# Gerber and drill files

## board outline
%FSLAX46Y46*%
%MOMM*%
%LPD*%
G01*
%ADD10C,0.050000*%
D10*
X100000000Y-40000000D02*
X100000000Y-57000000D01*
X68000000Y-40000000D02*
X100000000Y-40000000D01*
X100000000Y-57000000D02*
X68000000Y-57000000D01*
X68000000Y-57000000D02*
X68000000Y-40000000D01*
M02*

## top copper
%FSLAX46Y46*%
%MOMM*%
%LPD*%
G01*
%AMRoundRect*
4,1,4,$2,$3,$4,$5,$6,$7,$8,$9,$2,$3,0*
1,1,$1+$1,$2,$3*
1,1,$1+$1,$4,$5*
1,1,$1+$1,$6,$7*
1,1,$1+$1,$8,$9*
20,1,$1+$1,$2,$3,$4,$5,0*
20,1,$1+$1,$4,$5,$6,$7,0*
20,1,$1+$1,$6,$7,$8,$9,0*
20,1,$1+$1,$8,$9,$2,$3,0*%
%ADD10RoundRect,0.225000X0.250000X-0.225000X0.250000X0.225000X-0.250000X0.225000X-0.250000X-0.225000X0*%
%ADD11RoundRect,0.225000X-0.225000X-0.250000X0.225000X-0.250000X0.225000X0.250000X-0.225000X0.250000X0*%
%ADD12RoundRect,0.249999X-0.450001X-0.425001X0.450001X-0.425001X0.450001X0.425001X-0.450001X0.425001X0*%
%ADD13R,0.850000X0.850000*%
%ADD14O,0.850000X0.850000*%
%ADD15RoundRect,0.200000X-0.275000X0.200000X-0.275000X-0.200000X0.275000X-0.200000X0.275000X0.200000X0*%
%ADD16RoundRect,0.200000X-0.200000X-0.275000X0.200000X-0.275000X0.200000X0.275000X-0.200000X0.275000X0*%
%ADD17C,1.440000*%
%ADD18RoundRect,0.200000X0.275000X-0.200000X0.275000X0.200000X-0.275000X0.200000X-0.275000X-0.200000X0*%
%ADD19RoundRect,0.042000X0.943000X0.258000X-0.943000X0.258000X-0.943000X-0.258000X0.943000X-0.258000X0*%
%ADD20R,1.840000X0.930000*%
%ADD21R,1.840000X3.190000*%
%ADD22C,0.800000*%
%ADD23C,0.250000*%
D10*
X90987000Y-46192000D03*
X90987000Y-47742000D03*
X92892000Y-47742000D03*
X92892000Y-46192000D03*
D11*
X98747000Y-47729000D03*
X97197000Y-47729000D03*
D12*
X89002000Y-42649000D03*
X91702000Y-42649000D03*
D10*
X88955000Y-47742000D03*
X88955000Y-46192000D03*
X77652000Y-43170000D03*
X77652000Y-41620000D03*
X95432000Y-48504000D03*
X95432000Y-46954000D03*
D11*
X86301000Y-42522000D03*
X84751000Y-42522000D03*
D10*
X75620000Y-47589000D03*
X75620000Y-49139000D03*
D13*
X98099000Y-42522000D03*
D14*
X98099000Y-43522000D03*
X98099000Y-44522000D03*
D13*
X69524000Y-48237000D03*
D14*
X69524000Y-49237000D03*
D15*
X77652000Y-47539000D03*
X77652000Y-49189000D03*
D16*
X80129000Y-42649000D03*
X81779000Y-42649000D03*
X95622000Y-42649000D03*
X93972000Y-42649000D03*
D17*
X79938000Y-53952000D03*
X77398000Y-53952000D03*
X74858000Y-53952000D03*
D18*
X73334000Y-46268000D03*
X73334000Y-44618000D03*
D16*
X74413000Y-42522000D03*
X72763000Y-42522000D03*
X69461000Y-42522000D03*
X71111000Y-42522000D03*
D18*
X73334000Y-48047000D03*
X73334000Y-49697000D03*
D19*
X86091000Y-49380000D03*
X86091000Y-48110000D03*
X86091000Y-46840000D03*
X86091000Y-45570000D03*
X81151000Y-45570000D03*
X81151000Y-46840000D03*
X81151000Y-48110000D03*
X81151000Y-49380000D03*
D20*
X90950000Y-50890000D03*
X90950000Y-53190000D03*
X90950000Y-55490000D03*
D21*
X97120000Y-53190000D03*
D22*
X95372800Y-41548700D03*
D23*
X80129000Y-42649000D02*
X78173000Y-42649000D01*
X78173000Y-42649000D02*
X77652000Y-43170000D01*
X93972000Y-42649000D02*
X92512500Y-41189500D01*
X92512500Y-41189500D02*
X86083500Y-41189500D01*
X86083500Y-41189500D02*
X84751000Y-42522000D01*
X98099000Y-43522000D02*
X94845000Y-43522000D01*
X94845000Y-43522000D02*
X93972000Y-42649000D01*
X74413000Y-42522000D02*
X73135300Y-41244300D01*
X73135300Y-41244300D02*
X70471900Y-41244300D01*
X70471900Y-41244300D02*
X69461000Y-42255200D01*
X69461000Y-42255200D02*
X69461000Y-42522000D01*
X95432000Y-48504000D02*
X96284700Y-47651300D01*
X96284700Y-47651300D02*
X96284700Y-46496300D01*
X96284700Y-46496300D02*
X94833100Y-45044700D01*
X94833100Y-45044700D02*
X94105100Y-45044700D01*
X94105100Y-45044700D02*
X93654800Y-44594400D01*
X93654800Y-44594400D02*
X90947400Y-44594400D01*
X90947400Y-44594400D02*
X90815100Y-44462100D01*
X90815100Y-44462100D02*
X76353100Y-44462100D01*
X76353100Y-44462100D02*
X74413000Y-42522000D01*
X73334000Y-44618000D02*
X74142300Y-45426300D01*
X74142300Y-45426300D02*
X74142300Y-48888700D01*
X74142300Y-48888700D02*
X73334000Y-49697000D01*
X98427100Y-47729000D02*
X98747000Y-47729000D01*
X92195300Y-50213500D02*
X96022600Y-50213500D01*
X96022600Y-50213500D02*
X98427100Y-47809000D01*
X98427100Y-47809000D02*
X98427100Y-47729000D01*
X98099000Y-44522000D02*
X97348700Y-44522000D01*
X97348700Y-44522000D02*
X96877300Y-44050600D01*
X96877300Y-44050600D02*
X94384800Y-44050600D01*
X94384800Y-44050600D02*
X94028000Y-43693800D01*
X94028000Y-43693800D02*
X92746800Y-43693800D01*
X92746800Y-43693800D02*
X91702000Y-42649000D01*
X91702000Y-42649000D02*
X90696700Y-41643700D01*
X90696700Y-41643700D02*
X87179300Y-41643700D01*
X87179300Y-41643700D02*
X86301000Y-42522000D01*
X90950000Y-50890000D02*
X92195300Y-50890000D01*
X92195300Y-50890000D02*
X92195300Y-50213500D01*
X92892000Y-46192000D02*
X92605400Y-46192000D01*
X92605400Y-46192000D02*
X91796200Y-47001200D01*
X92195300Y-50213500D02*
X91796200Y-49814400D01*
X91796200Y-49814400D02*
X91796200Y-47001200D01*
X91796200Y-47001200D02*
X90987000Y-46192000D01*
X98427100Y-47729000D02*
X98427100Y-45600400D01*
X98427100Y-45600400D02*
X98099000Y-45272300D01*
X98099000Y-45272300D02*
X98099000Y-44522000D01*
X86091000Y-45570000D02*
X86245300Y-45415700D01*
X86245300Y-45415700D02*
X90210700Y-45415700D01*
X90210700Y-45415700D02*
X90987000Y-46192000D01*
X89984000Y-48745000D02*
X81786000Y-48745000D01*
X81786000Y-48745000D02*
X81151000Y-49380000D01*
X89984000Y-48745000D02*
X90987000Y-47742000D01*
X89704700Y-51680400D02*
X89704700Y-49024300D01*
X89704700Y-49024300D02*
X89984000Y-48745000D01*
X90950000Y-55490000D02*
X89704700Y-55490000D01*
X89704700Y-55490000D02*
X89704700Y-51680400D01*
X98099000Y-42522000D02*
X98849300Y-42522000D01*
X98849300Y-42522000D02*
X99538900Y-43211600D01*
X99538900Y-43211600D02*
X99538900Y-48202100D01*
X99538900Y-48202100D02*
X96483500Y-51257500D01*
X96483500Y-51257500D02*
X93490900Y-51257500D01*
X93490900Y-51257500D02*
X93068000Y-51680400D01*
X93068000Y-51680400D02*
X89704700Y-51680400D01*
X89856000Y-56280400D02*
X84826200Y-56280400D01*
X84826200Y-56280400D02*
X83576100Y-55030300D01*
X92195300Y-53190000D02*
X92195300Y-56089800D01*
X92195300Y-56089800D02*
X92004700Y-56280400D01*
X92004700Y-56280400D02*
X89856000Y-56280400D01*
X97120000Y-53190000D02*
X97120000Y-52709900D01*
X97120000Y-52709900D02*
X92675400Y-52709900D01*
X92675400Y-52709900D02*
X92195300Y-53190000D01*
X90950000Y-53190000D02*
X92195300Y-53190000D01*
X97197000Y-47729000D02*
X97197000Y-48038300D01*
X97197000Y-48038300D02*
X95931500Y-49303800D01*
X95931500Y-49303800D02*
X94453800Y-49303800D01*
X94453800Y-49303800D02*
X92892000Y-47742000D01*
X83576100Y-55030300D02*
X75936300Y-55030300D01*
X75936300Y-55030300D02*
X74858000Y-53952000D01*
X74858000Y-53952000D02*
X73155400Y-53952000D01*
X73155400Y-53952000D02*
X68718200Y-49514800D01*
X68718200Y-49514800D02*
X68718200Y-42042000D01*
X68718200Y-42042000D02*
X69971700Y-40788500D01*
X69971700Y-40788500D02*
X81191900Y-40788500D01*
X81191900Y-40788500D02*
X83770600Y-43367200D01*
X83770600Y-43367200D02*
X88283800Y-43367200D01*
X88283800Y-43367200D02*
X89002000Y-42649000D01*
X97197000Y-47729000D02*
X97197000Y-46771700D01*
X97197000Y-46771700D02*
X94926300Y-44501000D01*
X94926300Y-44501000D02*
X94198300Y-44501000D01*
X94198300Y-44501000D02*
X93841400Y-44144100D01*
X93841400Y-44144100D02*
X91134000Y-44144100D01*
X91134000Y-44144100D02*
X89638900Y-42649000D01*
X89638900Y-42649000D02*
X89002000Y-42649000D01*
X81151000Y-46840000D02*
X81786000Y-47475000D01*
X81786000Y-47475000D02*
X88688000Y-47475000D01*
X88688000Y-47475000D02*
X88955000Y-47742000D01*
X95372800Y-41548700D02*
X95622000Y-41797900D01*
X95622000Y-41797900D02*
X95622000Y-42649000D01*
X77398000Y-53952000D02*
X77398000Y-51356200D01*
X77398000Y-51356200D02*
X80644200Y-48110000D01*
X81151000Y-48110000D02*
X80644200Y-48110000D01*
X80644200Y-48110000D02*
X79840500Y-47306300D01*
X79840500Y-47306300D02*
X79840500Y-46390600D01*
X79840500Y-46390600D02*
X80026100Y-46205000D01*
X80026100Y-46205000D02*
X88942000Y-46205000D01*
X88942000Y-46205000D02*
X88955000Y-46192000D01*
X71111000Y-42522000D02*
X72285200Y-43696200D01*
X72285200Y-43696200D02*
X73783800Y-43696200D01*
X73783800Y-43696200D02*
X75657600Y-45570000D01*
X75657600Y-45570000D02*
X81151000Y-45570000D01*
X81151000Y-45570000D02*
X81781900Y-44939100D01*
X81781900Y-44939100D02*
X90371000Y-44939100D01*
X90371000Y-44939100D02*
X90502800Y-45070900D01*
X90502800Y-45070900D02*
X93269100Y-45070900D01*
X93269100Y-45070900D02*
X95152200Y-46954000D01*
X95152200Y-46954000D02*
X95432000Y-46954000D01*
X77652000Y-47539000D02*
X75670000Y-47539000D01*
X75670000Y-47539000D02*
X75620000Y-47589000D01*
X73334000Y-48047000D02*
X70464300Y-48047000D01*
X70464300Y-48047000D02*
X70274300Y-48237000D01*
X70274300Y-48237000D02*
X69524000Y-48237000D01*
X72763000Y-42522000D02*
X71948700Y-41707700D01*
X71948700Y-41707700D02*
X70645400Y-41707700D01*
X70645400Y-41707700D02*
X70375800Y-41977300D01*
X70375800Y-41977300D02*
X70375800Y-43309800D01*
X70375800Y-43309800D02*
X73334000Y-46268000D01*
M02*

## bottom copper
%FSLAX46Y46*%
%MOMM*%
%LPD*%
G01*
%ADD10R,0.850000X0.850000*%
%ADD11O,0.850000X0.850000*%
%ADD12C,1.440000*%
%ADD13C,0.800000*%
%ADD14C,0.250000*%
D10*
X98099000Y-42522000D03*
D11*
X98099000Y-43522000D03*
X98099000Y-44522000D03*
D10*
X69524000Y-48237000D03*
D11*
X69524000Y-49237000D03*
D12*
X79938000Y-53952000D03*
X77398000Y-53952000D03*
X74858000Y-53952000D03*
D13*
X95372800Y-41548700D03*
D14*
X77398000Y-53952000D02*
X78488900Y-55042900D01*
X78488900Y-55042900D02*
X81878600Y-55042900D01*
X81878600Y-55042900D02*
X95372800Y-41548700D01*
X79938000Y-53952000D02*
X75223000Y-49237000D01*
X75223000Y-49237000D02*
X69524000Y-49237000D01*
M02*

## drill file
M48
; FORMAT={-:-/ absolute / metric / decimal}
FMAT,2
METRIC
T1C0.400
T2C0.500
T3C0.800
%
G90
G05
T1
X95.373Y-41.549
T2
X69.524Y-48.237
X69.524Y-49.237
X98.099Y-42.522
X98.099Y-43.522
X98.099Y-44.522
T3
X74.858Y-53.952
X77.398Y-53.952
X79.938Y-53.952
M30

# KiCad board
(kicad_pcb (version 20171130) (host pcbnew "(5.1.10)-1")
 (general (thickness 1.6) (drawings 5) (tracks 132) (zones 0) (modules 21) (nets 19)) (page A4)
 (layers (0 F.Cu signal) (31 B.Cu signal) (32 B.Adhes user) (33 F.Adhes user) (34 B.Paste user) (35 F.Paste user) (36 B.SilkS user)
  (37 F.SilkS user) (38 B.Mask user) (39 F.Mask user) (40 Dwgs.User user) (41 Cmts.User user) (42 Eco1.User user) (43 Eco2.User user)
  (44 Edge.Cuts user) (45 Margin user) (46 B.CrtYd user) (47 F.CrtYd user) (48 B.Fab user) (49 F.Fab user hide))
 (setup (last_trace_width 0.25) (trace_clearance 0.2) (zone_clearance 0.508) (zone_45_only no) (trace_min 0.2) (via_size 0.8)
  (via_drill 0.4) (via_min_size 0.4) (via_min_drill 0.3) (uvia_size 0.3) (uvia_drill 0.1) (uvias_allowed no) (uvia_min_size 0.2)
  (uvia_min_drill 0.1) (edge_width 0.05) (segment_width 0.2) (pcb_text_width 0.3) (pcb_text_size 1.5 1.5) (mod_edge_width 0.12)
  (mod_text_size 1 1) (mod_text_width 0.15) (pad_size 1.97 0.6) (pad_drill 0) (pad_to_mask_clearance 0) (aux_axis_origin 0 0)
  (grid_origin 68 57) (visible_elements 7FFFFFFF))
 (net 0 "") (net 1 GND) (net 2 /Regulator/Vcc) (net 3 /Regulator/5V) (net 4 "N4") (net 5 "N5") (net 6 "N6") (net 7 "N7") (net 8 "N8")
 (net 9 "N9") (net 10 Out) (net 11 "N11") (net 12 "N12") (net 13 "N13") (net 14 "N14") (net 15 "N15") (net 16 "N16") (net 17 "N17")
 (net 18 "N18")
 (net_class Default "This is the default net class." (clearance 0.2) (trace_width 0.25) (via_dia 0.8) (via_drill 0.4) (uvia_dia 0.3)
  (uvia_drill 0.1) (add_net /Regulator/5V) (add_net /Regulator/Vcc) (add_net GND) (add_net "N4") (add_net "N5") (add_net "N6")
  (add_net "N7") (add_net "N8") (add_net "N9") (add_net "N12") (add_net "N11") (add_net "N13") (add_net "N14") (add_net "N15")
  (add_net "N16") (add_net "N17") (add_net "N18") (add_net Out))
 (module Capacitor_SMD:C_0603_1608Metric (layer F.Cu) (at 90.987 46.967 90)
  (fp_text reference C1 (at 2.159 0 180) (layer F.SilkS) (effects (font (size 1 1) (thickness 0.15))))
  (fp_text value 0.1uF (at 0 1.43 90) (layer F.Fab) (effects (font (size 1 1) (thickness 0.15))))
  (pad 2 smd roundrect (at 0.775 0 90) (size 0.9 0.95) (layers F.Cu F.Paste F.Mask) (roundrect_rratio 0.25) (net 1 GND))
  (pad 1 smd roundrect (at -0.775 0 90) (size 0.9 0.95) (layers F.Cu F.Paste F.Mask) (roundrect_rratio 0.25) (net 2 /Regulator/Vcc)))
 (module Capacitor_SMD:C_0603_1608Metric (layer F.Cu) (at 92.892 46.967 90)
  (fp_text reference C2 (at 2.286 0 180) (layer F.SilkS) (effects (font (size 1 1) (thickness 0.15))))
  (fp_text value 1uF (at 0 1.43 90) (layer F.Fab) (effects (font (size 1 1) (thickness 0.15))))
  (pad 1 smd roundrect (at -0.775 0 90) (size 0.9 0.95) (layers F.Cu F.Paste F.Mask) (roundrect_rratio 0.25) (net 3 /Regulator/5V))
  (pad 2 smd roundrect (at 0.775 0 90) (size 0.9 0.95) (layers F.Cu F.Paste F.Mask) (roundrect_rratio 0.25) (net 1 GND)))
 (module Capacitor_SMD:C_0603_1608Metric (layer F.Cu) (at 97.972 47.729)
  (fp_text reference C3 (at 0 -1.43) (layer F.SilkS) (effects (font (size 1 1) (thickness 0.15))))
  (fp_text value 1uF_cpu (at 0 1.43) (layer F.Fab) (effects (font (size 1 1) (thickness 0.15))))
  (pad 2 smd roundrect (at 0.775 0) (size 0.9 0.95) (layers F.Cu F.Paste F.Mask) (roundrect_rratio 0.25) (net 1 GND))
  (pad 1 smd roundrect (at -0.775 0) (size 0.9 0.95) (layers F.Cu F.Paste F.Mask) (roundrect_rratio 0.25) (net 3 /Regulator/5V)))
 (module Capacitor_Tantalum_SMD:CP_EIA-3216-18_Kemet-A (layer F.Cu) (at 90.352 42.649)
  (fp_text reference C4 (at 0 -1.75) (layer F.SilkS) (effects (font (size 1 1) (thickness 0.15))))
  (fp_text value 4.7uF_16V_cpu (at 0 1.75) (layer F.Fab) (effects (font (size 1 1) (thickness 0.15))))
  (pad 1 smd roundrect (at -1.35 0) (size 1.4 1.35) (layers F.Cu F.Paste F.Mask) (roundrect_rratio 0.1851844444444445) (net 3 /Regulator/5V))
  (pad 2 smd roundrect (at 1.35 0) (size 1.4 1.35) (layers F.Cu F.Paste F.Mask) (roundrect_rratio 0.1851844444444445) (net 1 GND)))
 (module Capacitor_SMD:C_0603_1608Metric (layer F.Cu) (at 88.955 46.967 90)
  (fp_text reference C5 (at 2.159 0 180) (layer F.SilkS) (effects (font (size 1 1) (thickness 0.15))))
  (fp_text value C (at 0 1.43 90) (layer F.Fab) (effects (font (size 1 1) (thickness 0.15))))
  (pad 1 smd roundrect (at -0.775 0 90) (size 0.9 0.95) (layers F.Cu F.Paste F.Mask) (roundrect_rratio 0.25) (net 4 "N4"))
  (pad 2 smd roundrect (at 0.775 0 90) (size 0.9 0.95) (layers F.Cu F.Paste F.Mask) (roundrect_rratio 0.25) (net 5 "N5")))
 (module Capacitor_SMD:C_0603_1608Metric (layer F.Cu) (at 77.652 42.395 90)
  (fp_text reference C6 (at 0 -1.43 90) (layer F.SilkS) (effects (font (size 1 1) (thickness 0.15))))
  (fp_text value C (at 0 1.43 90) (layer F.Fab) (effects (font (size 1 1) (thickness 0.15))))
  (pad 1 smd roundrect (at -0.775 0 90) (size 0.9 0.95) (layers F.Cu F.Paste F.Mask) (roundrect_rratio 0.25) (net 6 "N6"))
  (pad 2 smd roundrect (at 0.775 0 90) (size 0.9 0.95) (layers F.Cu F.Paste F.Mask) (roundrect_rratio 0.25) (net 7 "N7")))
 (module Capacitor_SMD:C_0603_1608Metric (layer F.Cu) (at 95.432 47.729 90)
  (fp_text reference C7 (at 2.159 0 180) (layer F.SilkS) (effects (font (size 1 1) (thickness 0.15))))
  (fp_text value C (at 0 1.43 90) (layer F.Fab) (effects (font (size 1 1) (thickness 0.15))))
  (pad 1 smd roundrect (at -0.775 0 90) (size 0.9 0.95) (layers F.Cu F.Paste F.Mask) (roundrect_rratio 0.25) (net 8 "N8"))
  (pad 2 smd roundrect (at 0.775 0 90) (size 0.9 0.95) (layers F.Cu F.Paste F.Mask) (roundrect_rratio 0.25) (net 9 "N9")))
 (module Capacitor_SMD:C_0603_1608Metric (layer F.Cu) (at 85.526 42.522)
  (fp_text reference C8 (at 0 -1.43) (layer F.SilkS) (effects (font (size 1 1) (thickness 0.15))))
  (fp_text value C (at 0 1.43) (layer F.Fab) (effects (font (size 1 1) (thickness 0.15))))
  (pad 2 smd roundrect (at 0.775 0) (size 0.9 0.95) (layers F.Cu F.Paste F.Mask) (roundrect_rratio 0.25) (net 1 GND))
  (pad 1 smd roundrect (at -0.775 0) (size 0.9 0.95) (layers F.Cu F.Paste F.Mask) (roundrect_rratio 0.25) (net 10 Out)))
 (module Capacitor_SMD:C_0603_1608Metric (layer F.Cu) (at 75.62 48.364 90)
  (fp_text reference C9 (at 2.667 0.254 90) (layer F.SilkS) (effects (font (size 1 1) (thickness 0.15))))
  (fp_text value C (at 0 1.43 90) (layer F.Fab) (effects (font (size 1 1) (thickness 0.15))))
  (pad 2 smd roundrect (at 0.775 0 90) (size 0.9 0.95) (layers F.Cu F.Paste F.Mask) (roundrect_rratio 0.25) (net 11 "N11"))
  (pad 1 smd roundrect (at -0.775 0 90) (size 0.9 0.95) (layers F.Cu F.Paste F.Mask) (roundrect_rratio 0.25) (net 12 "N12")))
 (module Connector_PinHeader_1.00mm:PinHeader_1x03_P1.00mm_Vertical (layer F.Cu) (at 98.099 42.522)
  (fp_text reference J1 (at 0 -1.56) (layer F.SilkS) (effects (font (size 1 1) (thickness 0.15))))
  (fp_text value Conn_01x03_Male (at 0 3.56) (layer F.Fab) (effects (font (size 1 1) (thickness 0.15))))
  (pad 1 thru_hole rect (at 0 0) (size 0.85 0.85) (drill 0.5) (layers *.Cu *.Mask) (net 2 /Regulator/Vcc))
  (pad 2 thru_hole oval (at 0 1) (size 0.85 0.85) (drill 0.5) (layers *.Cu *.Mask) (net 10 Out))
  (pad 3 thru_hole oval (at 0 2) (size 0.85 0.85) (drill 0.5) (layers *.Cu *.Mask) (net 1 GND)))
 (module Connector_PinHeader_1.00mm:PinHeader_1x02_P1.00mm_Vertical (layer F.Cu) (at 69.524 48.237)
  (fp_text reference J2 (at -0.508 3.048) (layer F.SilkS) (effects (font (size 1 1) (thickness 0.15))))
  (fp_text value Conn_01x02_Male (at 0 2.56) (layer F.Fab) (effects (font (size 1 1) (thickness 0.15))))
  (pad 1 thru_hole rect (at 0 0) (size 0.85 0.85) (drill 0.5) (layers *.Cu *.Mask) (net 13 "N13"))
  (pad 2 thru_hole oval (at 0 1) (size 0.85 0.85) (drill 0.5) (layers *.Cu *.Mask) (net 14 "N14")))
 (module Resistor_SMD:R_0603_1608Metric (layer F.Cu) (at 77.652 48.364 270)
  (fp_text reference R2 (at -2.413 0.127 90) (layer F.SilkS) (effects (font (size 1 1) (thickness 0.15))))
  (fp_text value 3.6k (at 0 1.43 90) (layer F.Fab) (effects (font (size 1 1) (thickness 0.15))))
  (pad 1 smd roundrect (at -0.825 0 270) (size 0.8 0.95) (layers F.Cu F.Paste F.Mask) (roundrect_rratio 0.25) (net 11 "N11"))
  (pad 2 smd roundrect (at 0.825 0 270) (size 0.8 0.95) (layers F.Cu F.Paste F.Mask) (roundrect_rratio 0.25) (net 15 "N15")))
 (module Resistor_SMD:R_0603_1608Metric (layer F.Cu) (at 80.954 42.649)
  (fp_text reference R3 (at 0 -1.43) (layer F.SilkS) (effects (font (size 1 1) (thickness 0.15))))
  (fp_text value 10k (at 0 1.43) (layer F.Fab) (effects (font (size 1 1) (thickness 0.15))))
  (pad 1 smd roundrect (at -0.825 0) (size 0.8 0.95) (layers F.Cu F.Paste F.Mask) (roundrect_rratio 0.25) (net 6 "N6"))
  (pad 2 smd roundrect (at 0.825 0) (size 0.8 0.95) (layers F.Cu F.Paste F.Mask) (roundrect_rratio 0.25) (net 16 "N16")))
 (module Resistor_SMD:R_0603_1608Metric (layer F.Cu) (at 94.797 42.649)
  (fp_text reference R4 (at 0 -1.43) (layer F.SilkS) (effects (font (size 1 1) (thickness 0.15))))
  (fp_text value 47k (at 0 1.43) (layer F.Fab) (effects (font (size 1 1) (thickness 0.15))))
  (pad 2 smd roundrect (at 0.825 0) (size 0.8 0.95) (layers F.Cu F.Paste F.Mask) (roundrect_rratio 0.25) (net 5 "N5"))
  (pad 1 smd roundrect (at -0.825 0) (size 0.8 0.95) (layers F.Cu F.Paste F.Mask) (roundrect_rratio 0.25) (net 10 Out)))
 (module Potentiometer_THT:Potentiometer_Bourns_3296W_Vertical (layer F.Cu) (at 79.938 53.952)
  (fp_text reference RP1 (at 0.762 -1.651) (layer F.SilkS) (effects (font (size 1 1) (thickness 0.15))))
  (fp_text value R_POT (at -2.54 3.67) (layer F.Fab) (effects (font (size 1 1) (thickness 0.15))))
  (pad 1 thru_hole circle (at 0 0) (size 1.44 1.44) (drill 0.8) (layers *.Cu *.Mask) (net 14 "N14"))
  (pad 2 thru_hole circle (at -2.54 0) (size 1.44 1.44) (drill 0.8) (layers *.Cu *.Mask) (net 5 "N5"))
  (pad 3 thru_hole circle (at -5.08 0) (size 1.44 1.44) (drill 0.8) (layers *.Cu *.Mask) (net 3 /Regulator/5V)))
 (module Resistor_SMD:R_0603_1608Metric (layer F.Cu) (at 73.334 45.443 90)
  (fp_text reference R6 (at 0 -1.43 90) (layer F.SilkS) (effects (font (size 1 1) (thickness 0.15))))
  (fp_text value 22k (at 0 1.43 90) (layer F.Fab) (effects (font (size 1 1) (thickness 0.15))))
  (pad 1 smd roundrect (at -0.825 0 90) (size 0.8 0.95) (layers F.Cu F.Paste F.Mask) (roundrect_rratio 0.25) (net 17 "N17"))
  (pad 2 smd roundrect (at 0.825 0 90) (size 0.8 0.95) (layers F.Cu F.Paste F.Mask) (roundrect_rratio 0.25) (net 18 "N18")))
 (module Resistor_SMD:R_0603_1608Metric (layer F.Cu) (at 73.588 42.522)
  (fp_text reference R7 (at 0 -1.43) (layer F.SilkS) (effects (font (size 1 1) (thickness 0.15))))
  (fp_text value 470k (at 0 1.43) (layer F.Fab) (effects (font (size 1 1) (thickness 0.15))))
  (pad 2 smd roundrect (at 0.825 0) (size 0.8 0.95) (layers F.Cu F.Paste F.Mask) (roundrect_rratio 0.25) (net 8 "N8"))
  (pad 1 smd roundrect (at -0.825 0) (size 0.8 0.95) (layers F.Cu F.Paste F.Mask) (roundrect_rratio 0.25) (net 17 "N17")))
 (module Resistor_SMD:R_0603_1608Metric (layer F.Cu) (at 70.286 42.522)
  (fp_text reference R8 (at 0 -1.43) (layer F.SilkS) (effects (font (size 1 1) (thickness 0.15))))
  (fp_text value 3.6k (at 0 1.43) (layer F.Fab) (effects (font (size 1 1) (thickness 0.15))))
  (pad 1 smd roundrect (at -0.825 0) (size 0.8 0.95) (layers F.Cu F.Paste F.Mask) (roundrect_rratio 0.25) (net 8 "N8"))
  (pad 2 smd roundrect (at 0.825 0) (size 0.8 0.95) (layers F.Cu F.Paste F.Mask) (roundrect_rratio 0.25) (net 9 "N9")))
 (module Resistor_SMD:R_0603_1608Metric (layer F.Cu) (at 73.334 48.872 90)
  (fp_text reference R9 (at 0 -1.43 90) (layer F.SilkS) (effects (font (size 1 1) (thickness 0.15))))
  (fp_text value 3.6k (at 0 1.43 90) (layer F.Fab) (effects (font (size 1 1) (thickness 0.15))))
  (pad 2 smd roundrect (at 0.825 0 90) (size 0.8 0.95) (layers F.Cu F.Paste F.Mask) (roundrect_rratio 0.25) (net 13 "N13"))
  (pad 1 smd roundrect (at -0.825 0 90) (size 0.8 0.95) (layers F.Cu F.Paste F.Mask) (roundrect_rratio 0.25) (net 18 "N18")))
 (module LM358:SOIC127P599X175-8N (layer F.Cu) (at 83.621 47.475 180)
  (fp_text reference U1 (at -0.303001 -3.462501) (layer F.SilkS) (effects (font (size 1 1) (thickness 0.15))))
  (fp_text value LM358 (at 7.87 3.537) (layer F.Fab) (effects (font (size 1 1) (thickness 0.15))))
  (pad 1 smd roundrect (at -2.47 -1.905 180) (size 1.97 0.6) (layers F.Cu F.Paste F.Mask) (roundrect_rratio 0.07000000000000001))
  (pad 2 smd roundrect (at -2.47 -0.635 180) (size 1.97 0.6) (layers F.Cu F.Paste F.Mask) (roundrect_rratio 0.07000000000000001))
  (pad 3 smd roundrect (at -2.47 0.635 180) (size 1.97 0.6) (layers F.Cu F.Paste F.Mask) (roundrect_rratio 0.07000000000000001))
  (pad 4 smd roundrect (at -2.47 1.905 180) (size 1.97 0.6) (layers F.Cu F.Paste F.Mask) (roundrect_rratio 0.07000000000000001) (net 1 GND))
  (pad 5 smd roundrect (at 2.47 1.905 180) (size 1.97 0.6) (layers F.Cu F.Paste F.Mask) (roundrect_rratio 0.07000000000000001) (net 9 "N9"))
  (pad 6 smd roundrect (at 2.47 0.635 180) (size 1.97 0.6) (layers F.Cu F.Paste F.Mask) (roundrect_rratio 0.07000000000000001) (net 4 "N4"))
  (pad 7 smd roundrect (at 2.47 -0.635 180) (size 1.97 0.6) (layers F.Cu F.Paste F.Mask) (roundrect_rratio 0.07000000000000001) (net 5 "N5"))
  (pad 8 smd roundrect (at 2.47 -1.905 180) (size 1.97 0.6) (layers F.Cu F.Paste F.Mask) (roundrect_rratio 0.07000000000000001)
   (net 2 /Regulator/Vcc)))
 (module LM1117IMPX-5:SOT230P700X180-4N (layer F.Cu) (at 94.035 53.19)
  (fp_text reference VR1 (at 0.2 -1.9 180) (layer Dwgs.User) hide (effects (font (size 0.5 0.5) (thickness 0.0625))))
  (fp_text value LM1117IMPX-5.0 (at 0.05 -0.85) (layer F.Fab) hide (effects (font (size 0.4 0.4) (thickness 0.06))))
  (pad 1 smd rect (at -3.085 -2.3) (size 1.84 0.93) (layers F.Cu F.Paste F.Mask) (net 1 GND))
  (pad 2 smd rect (at -3.085 0) (size 1.84 0.93) (layers F.Cu F.Paste F.Mask) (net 3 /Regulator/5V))
  (pad 3 smd rect (at -3.085 2.3) (size 1.84 0.93) (layers F.Cu F.Paste F.Mask) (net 2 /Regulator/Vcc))
  (pad 4 smd rect (at 3.085 0) (size 1.84 3.19) (layers F.Cu F.Paste F.Mask) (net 3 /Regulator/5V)))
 (gr_line (start 100 40) (end 100 57) (layer Edge.Cuts) (width 0.05))
 (gr_line (start 68 40) (end 100 40) (layer Edge.Cuts) (width 0.05))
 (gr_line (start 100 57) (end 68 57) (layer Edge.Cuts) (width 0.05))
 (gr_line (start 68 57) (end 68 40) (layer Edge.Cuts) (width 0.05))
 (segment (start 80.129 42.649) (end 78.173 42.649) (width 0.25) (layer F.Cu) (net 6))
 (segment (start 78.173 42.649) (end 77.652 43.17) (width 0.25) (layer F.Cu) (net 6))
 (segment (start 93.972 42.649) (end 92.5125 41.1895) (width 0.25) (layer F.Cu) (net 10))
 (segment (start 92.5125 41.1895) (end 86.0835 41.1895) (width 0.25) (layer F.Cu) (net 10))
 (segment (start 86.0835 41.1895) (end 84.751 42.522) (width 0.25) (layer F.Cu) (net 10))
 (segment (start 98.099 43.522) (end 94.845 43.522) (width 0.25) (layer F.Cu) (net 10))
 (segment (start 94.845 43.522) (end 93.972 42.649) (width 0.25) (layer F.Cu) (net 10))
 (segment (start 74.413 42.522) (end 73.1353 41.2443) (width 0.25) (layer F.Cu) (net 8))
 (segment (start 73.1353 41.2443) (end 70.4719 41.2443) (width 0.25) (layer F.Cu) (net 8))
 (segment (start 70.4719 41.2443) (end 69.461 42.2552) (width 0.25) (layer F.Cu) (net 8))
 (segment (start 69.461 42.2552) (end 69.461 42.522) (width 0.25) (layer F.Cu) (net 8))
 (segment (start 95.432 48.504) (end 96.2847 47.6513) (width 0.25) (layer F.Cu) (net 8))
 (segment (start 96.2847 47.6513) (end 96.2847 46.4963) (width 0.25) (layer F.Cu) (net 8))
 (segment (start 96.2847 46.4963) (end 94.8331 45.0447) (width 0.25) (layer F.Cu) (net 8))
 (segment (start 94.8331 45.0447) (end 94.1051 45.0447) (width 0.25) (layer F.Cu) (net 8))
 (segment (start 94.1051 45.0447) (end 93.6548 44.5944) (width 0.25) (layer F.Cu) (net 8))
 (segment (start 93.6548 44.5944) (end 90.9474 44.5944) (width 0.25) (layer F.Cu) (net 8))
 (segment (start 90.9474 44.5944) (end 90.8151 44.4621) (width 0.25) (layer F.Cu) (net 8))
 (segment (start 90.8151 44.4621) (end 76.3531 44.4621) (width 0.25) (layer F.Cu) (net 8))
 (segment (start 76.3531 44.4621) (end 74.413 42.522) (width 0.25) (layer F.Cu) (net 8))
 (segment (start 73.334 44.618) (end 74.1423 45.4263) (width 0.25) (layer F.Cu) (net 18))
 (segment (start 74.1423 45.4263) (end 74.1423 48.8887) (width 0.25) (layer F.Cu) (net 18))
 (segment (start 74.1423 48.8887) (end 73.334 49.697) (width 0.25) (layer F.Cu) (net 18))
 (segment (start 98.4271 47.729) (end 98.747 47.729) (width 0.25) (layer F.Cu) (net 1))
 (segment (start 92.1953 50.2135) (end 96.0226 50.2135) (width 0.25) (layer F.Cu) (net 1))
 (segment (start 96.0226 50.2135) (end 98.4271 47.809) (width 0.25) (layer F.Cu) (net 1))
 (segment (start 98.4271 47.809) (end 98.4271 47.729) (width 0.25) (layer F.Cu) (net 1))
 (segment (start 98.099 44.522) (end 97.3487 44.522) (width 0.25) (layer F.Cu) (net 1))
 (segment (start 97.3487 44.522) (end 96.8773 44.0506) (width 0.25) (layer F.Cu) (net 1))
 (segment (start 96.8773 44.0506) (end 94.3848 44.0506) (width 0.25) (layer F.Cu) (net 1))
 (segment (start 94.3848 44.0506) (end 94.028 43.6938) (width 0.25) (layer F.Cu) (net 1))
 (segment (start 94.028 43.6938) (end 92.7468 43.6938) (width 0.25) (layer F.Cu) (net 1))
 (segment (start 92.7468 43.6938) (end 91.702 42.649) (width 0.25) (layer F.Cu) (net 1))
 (segment (start 91.702 42.649) (end 90.6967 41.6437) (width 0.25) (layer F.Cu) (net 1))
 (segment (start 90.6967 41.6437) (end 87.1793 41.6437) (width 0.25) (layer F.Cu) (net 1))
 (segment (start 87.1793 41.6437) (end 86.301 42.522) (width 0.25) (layer F.Cu) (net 1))
 (segment (start 90.95 50.89) (end 92.1953 50.89) (width 0.25) (layer F.Cu) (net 1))
 (segment (start 92.1953 50.89) (end 92.1953 50.2135) (width 0.25) (layer F.Cu) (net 1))
 (segment (start 92.892 46.192) (end 92.6054 46.192) (width 0.25) (layer F.Cu) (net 1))
 (segment (start 92.6054 46.192) (end 91.7962 47.0012) (width 0.25) (layer F.Cu) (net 1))
 (segment (start 92.1953 50.2135) (end 91.7962 49.8144) (width 0.25) (layer F.Cu) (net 1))
 (segment (start 91.7962 49.8144) (end 91.7962 47.0012) (width 0.25) (layer F.Cu) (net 1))
 (segment (start 91.7962 47.0012) (end 90.987 46.192) (width 0.25) (layer F.Cu) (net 1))
 (segment (start 98.4271 47.729) (end 98.4271 45.6004) (width 0.25) (layer F.Cu) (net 1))
 (segment (start 98.4271 45.6004) (end 98.099 45.2723) (width 0.25) (layer F.Cu) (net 1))
 (segment (start 98.099 45.2723) (end 98.099 44.522) (width 0.25) (layer F.Cu) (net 1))
 (segment (start 86.091 45.57) (end 86.2453 45.4157) (width 0.25) (layer F.Cu) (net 1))
 (segment (start 86.2453 45.4157) (end 90.2107 45.4157) (width 0.25) (layer F.Cu) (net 1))
 (segment (start 90.2107 45.4157) (end 90.987 46.192) (width 0.25) (layer F.Cu) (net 1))
 (segment (start 89.984 48.745) (end 81.786 48.745) (width 0.25) (layer F.Cu) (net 2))
 (segment (start 81.786 48.745) (end 81.151 49.38) (width 0.25) (layer F.Cu) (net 2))
 (segment (start 89.984 48.745) (end 90.987 47.742) (width 0.25) (layer F.Cu) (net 2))
 (segment (start 89.7047 51.6804) (end 89.7047 49.0243) (width 0.25) (layer F.Cu) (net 2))
 (segment (start 89.7047 49.0243) (end 89.984 48.745) (width 0.25) (layer F.Cu) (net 2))
 (segment (start 90.95 55.49) (end 89.7047 55.49) (width 0.25) (layer F.Cu) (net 2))
 (segment (start 89.7047 55.49) (end 89.7047 51.6804) (width 0.25) (layer F.Cu) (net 2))
 (segment (start 98.099 42.522) (end 98.8493 42.522) (width 0.25) (layer F.Cu) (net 2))
 (segment (start 98.8493 42.522) (end 99.5389 43.2116) (width 0.25) (layer F.Cu) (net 2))
 (segment (start 99.5389 43.2116) (end 99.5389 48.2021) (width 0.25) (layer F.Cu) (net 2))
 (segment (start 99.5389 48.2021) (end 96.4835 51.2575) (width 0.25) (layer F.Cu) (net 2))
 (segment (start 96.4835 51.2575) (end 93.4909 51.2575) (width 0.25) (layer F.Cu) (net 2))
 (segment (start 93.4909 51.2575) (end 93.068 51.6804) (width 0.25) (layer F.Cu) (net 2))
 (segment (start 93.068 51.6804) (end 89.7047 51.6804) (width 0.25) (layer F.Cu) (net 2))
 (segment (start 89.856 56.2804) (end 84.8262 56.2804) (width 0.25) (layer F.Cu) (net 3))
 (segment (start 84.8262 56.2804) (end 83.5761 55.0303) (width 0.25) (layer F.Cu) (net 3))
 (segment (start 92.1953 53.19) (end 92.1953 56.0898) (width 0.25) (layer F.Cu) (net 3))
 (segment (start 92.1953 56.0898) (end 92.0047 56.2804) (width 0.25) (layer F.Cu) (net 3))
 (segment (start 92.0047 56.2804) (end 89.856 56.2804) (width 0.25) (layer F.Cu) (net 3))
 (segment (start 97.12 53.19) (end 97.12 52.7099) (width 0.25) (layer F.Cu) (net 3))
 (segment (start 97.12 52.7099) (end 92.6754 52.7099) (width 0.25) (layer F.Cu) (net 3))
 (segment (start 92.6754 52.7099) (end 92.1953 53.19) (width 0.25) (layer F.Cu) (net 3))
 (segment (start 90.95 53.19) (end 92.1953 53.19) (width 0.25) (layer F.Cu) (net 3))
 (segment (start 97.197 47.729) (end 97.197 48.0383) (width 0.25) (layer F.Cu) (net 3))
 (segment (start 97.197 48.0383) (end 95.9315 49.3038) (width 0.25) (layer F.Cu) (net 3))
 (segment (start 95.9315 49.3038) (end 94.4538 49.3038) (width 0.25) (layer F.Cu) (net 3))
 (segment (start 94.4538 49.3038) (end 92.892 47.742) (width 0.25) (layer F.Cu) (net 3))
 (segment (start 83.5761 55.0303) (end 75.9363 55.0303) (width 0.25) (layer F.Cu) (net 3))
 (segment (start 75.9363 55.0303) (end 74.858 53.952) (width 0.25) (layer F.Cu) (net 3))
 (segment (start 74.858 53.952) (end 73.1554 53.952) (width 0.25) (layer F.Cu) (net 3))
 (segment (start 73.1554 53.952) (end 68.7182 49.5148) (width 0.25) (layer F.Cu) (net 3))
 (segment (start 68.7182 49.5148) (end 68.7182 42.042) (width 0.25) (layer F.Cu) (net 3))
 (segment (start 68.7182 42.042) (end 69.9717 40.7885) (width 0.25) (layer F.Cu) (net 3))
 (segment (start 69.9717 40.7885) (end 81.1919 40.7885) (width 0.25) (layer F.Cu) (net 3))
 (segment (start 81.1919 40.7885) (end 83.7706 43.3672) (width 0.25) (layer F.Cu) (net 3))
 (segment (start 83.7706 43.3672) (end 88.2838 43.3672) (width 0.25) (layer F.Cu) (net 3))
 (segment (start 88.2838 43.3672) (end 89.002 42.649) (width 0.25) (layer F.Cu) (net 3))
 (segment (start 97.197 47.729) (end 97.197 46.7717) (width 0.25) (layer F.Cu) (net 3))
 (segment (start 97.197 46.7717) (end 94.9263 44.501) (width 0.25) (layer F.Cu) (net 3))
 (segment (start 94.9263 44.501) (end 94.1983 44.501) (width 0.25) (layer F.Cu) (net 3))
 (segment (start 94.1983 44.501) (end 93.8414 44.1441) (width 0.25) (layer F.Cu) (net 3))
 (segment (start 93.8414 44.1441) (end 91.134 44.1441) (width 0.25) (layer F.Cu) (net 3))
 (segment (start 91.134 44.1441) (end 89.6389 42.649) (width 0.25) (layer F.Cu) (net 3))
 (segment (start 89.6389 42.649) (end 89.002 42.649) (width 0.25) (layer F.Cu) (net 3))
 (segment (start 81.151 46.84) (end 81.786 47.475) (width 0.25) (layer F.Cu) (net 4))
 (segment (start 81.786 47.475) (end 88.688 47.475) (width 0.25) (layer F.Cu) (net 4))
 (segment (start 88.688 47.475) (end 88.955 47.742) (width 0.25) (layer F.Cu) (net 4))
 (segment (start 77.398 53.952) (end 78.4889 55.0429) (width 0.25) (layer B.Cu) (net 5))
 (segment (start 78.4889 55.0429) (end 81.8786 55.0429) (width 0.25) (layer B.Cu) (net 5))
 (segment (start 81.8786 55.0429) (end 95.3728 41.5487) (width 0.25) (layer B.Cu) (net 5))
 (segment (start 95.3728 41.5487) (end 95.622 41.7979) (width 0.25) (layer F.Cu) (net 5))
 (segment (start 95.622 41.7979) (end 95.622 42.649) (width 0.25) (layer F.Cu) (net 5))
 (segment (start 77.398 53.952) (end 77.398 51.3562) (width 0.25) (layer F.Cu) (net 5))
 (segment (start 77.398 51.3562) (end 80.6442 48.11) (width 0.25) (layer F.Cu) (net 5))
 (segment (start 81.151 48.11) (end 80.6442 48.11) (width 0.25) (layer F.Cu) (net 5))
 (segment (start 80.6442 48.11) (end 79.8405 47.3063) (width 0.25) (layer F.Cu) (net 5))
 (segment (start 79.8405 47.3063) (end 79.8405 46.3906) (width 0.25) (layer F.Cu) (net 5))
 (segment (start 79.8405 46.3906) (end 80.0261 46.205) (width 0.25) (layer F.Cu) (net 5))
 (segment (start 80.0261 46.205) (end 88.942 46.205) (width 0.25) (layer F.Cu) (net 5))
 (segment (start 88.942 46.205) (end 88.955 46.192) (width 0.25) (layer F.Cu) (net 5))
 (via (at 95.3728 41.5487) (size 0.8) (layers F.Cu B.Cu) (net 5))
 (segment (start 71.111 42.522) (end 72.2852 43.6962) (width 0.25) (layer F.Cu) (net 9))
 (segment (start 72.2852 43.6962) (end 73.7838 43.6962) (width 0.25) (layer F.Cu) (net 9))
 (segment (start 73.7838 43.6962) (end 75.6576 45.57) (width 0.25) (layer F.Cu) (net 9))
 (segment (start 75.6576 45.57) (end 81.151 45.57) (width 0.25) (layer F.Cu) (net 9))
 (segment (start 81.151 45.57) (end 81.7819 44.9391) (width 0.25) (layer F.Cu) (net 9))
 (segment (start 81.7819 44.9391) (end 90.371 44.9391) (width 0.25) (layer F.Cu) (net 9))
 (segment (start 90.371 44.9391) (end 90.5028 45.0709) (width 0.25) (layer F.Cu) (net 9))
 (segment (start 90.5028 45.0709) (end 93.2691 45.0709) (width 0.25) (layer F.Cu) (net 9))
 (segment (start 93.2691 45.0709) (end 95.1522 46.954) (width 0.25) (layer F.Cu) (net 9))
 (segment (start 95.1522 46.954) (end 95.432 46.954) (width 0.25) (layer F.Cu) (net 9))
 (segment (start 77.652 47.539) (end 75.67 47.539) (width 0.25) (layer F.Cu) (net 11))
 (segment (start 75.67 47.539) (end 75.62 47.589) (width 0.25) (layer F.Cu) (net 11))
 (segment (start 73.334 48.047) (end 70.4643 48.047) (width 0.25) (layer F.Cu) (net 13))
 (segment (start 70.4643 48.047) (end 70.2743 48.237) (width 0.25) (layer F.Cu) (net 13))
 (segment (start 70.2743 48.237) (end 69.524 48.237) (width 0.25) (layer F.Cu) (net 13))
 (segment (start 79.938 53.952) (end 75.223 49.237) (width 0.25) (layer B.Cu) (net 14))
 (segment (start 75.223 49.237) (end 69.524 49.237) (width 0.25) (layer B.Cu) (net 14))
 (segment (start 72.763 42.522) (end 71.9487 41.7077) (width 0.25) (layer F.Cu) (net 17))
 (segment (start 71.9487 41.7077) (end 70.6454 41.7077) (width 0.25) (layer F.Cu) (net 17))
 (segment (start 70.6454 41.7077) (end 70.3758 41.9773) (width 0.25) (layer F.Cu) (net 17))
 (segment (start 70.3758 41.9773) (end 70.3758 43.3098) (width 0.25) (layer F.Cu) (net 17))
 (segment (start 70.3758 43.3098) (end 73.334 46.268) (width 0.25) (layer F.Cu) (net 17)))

